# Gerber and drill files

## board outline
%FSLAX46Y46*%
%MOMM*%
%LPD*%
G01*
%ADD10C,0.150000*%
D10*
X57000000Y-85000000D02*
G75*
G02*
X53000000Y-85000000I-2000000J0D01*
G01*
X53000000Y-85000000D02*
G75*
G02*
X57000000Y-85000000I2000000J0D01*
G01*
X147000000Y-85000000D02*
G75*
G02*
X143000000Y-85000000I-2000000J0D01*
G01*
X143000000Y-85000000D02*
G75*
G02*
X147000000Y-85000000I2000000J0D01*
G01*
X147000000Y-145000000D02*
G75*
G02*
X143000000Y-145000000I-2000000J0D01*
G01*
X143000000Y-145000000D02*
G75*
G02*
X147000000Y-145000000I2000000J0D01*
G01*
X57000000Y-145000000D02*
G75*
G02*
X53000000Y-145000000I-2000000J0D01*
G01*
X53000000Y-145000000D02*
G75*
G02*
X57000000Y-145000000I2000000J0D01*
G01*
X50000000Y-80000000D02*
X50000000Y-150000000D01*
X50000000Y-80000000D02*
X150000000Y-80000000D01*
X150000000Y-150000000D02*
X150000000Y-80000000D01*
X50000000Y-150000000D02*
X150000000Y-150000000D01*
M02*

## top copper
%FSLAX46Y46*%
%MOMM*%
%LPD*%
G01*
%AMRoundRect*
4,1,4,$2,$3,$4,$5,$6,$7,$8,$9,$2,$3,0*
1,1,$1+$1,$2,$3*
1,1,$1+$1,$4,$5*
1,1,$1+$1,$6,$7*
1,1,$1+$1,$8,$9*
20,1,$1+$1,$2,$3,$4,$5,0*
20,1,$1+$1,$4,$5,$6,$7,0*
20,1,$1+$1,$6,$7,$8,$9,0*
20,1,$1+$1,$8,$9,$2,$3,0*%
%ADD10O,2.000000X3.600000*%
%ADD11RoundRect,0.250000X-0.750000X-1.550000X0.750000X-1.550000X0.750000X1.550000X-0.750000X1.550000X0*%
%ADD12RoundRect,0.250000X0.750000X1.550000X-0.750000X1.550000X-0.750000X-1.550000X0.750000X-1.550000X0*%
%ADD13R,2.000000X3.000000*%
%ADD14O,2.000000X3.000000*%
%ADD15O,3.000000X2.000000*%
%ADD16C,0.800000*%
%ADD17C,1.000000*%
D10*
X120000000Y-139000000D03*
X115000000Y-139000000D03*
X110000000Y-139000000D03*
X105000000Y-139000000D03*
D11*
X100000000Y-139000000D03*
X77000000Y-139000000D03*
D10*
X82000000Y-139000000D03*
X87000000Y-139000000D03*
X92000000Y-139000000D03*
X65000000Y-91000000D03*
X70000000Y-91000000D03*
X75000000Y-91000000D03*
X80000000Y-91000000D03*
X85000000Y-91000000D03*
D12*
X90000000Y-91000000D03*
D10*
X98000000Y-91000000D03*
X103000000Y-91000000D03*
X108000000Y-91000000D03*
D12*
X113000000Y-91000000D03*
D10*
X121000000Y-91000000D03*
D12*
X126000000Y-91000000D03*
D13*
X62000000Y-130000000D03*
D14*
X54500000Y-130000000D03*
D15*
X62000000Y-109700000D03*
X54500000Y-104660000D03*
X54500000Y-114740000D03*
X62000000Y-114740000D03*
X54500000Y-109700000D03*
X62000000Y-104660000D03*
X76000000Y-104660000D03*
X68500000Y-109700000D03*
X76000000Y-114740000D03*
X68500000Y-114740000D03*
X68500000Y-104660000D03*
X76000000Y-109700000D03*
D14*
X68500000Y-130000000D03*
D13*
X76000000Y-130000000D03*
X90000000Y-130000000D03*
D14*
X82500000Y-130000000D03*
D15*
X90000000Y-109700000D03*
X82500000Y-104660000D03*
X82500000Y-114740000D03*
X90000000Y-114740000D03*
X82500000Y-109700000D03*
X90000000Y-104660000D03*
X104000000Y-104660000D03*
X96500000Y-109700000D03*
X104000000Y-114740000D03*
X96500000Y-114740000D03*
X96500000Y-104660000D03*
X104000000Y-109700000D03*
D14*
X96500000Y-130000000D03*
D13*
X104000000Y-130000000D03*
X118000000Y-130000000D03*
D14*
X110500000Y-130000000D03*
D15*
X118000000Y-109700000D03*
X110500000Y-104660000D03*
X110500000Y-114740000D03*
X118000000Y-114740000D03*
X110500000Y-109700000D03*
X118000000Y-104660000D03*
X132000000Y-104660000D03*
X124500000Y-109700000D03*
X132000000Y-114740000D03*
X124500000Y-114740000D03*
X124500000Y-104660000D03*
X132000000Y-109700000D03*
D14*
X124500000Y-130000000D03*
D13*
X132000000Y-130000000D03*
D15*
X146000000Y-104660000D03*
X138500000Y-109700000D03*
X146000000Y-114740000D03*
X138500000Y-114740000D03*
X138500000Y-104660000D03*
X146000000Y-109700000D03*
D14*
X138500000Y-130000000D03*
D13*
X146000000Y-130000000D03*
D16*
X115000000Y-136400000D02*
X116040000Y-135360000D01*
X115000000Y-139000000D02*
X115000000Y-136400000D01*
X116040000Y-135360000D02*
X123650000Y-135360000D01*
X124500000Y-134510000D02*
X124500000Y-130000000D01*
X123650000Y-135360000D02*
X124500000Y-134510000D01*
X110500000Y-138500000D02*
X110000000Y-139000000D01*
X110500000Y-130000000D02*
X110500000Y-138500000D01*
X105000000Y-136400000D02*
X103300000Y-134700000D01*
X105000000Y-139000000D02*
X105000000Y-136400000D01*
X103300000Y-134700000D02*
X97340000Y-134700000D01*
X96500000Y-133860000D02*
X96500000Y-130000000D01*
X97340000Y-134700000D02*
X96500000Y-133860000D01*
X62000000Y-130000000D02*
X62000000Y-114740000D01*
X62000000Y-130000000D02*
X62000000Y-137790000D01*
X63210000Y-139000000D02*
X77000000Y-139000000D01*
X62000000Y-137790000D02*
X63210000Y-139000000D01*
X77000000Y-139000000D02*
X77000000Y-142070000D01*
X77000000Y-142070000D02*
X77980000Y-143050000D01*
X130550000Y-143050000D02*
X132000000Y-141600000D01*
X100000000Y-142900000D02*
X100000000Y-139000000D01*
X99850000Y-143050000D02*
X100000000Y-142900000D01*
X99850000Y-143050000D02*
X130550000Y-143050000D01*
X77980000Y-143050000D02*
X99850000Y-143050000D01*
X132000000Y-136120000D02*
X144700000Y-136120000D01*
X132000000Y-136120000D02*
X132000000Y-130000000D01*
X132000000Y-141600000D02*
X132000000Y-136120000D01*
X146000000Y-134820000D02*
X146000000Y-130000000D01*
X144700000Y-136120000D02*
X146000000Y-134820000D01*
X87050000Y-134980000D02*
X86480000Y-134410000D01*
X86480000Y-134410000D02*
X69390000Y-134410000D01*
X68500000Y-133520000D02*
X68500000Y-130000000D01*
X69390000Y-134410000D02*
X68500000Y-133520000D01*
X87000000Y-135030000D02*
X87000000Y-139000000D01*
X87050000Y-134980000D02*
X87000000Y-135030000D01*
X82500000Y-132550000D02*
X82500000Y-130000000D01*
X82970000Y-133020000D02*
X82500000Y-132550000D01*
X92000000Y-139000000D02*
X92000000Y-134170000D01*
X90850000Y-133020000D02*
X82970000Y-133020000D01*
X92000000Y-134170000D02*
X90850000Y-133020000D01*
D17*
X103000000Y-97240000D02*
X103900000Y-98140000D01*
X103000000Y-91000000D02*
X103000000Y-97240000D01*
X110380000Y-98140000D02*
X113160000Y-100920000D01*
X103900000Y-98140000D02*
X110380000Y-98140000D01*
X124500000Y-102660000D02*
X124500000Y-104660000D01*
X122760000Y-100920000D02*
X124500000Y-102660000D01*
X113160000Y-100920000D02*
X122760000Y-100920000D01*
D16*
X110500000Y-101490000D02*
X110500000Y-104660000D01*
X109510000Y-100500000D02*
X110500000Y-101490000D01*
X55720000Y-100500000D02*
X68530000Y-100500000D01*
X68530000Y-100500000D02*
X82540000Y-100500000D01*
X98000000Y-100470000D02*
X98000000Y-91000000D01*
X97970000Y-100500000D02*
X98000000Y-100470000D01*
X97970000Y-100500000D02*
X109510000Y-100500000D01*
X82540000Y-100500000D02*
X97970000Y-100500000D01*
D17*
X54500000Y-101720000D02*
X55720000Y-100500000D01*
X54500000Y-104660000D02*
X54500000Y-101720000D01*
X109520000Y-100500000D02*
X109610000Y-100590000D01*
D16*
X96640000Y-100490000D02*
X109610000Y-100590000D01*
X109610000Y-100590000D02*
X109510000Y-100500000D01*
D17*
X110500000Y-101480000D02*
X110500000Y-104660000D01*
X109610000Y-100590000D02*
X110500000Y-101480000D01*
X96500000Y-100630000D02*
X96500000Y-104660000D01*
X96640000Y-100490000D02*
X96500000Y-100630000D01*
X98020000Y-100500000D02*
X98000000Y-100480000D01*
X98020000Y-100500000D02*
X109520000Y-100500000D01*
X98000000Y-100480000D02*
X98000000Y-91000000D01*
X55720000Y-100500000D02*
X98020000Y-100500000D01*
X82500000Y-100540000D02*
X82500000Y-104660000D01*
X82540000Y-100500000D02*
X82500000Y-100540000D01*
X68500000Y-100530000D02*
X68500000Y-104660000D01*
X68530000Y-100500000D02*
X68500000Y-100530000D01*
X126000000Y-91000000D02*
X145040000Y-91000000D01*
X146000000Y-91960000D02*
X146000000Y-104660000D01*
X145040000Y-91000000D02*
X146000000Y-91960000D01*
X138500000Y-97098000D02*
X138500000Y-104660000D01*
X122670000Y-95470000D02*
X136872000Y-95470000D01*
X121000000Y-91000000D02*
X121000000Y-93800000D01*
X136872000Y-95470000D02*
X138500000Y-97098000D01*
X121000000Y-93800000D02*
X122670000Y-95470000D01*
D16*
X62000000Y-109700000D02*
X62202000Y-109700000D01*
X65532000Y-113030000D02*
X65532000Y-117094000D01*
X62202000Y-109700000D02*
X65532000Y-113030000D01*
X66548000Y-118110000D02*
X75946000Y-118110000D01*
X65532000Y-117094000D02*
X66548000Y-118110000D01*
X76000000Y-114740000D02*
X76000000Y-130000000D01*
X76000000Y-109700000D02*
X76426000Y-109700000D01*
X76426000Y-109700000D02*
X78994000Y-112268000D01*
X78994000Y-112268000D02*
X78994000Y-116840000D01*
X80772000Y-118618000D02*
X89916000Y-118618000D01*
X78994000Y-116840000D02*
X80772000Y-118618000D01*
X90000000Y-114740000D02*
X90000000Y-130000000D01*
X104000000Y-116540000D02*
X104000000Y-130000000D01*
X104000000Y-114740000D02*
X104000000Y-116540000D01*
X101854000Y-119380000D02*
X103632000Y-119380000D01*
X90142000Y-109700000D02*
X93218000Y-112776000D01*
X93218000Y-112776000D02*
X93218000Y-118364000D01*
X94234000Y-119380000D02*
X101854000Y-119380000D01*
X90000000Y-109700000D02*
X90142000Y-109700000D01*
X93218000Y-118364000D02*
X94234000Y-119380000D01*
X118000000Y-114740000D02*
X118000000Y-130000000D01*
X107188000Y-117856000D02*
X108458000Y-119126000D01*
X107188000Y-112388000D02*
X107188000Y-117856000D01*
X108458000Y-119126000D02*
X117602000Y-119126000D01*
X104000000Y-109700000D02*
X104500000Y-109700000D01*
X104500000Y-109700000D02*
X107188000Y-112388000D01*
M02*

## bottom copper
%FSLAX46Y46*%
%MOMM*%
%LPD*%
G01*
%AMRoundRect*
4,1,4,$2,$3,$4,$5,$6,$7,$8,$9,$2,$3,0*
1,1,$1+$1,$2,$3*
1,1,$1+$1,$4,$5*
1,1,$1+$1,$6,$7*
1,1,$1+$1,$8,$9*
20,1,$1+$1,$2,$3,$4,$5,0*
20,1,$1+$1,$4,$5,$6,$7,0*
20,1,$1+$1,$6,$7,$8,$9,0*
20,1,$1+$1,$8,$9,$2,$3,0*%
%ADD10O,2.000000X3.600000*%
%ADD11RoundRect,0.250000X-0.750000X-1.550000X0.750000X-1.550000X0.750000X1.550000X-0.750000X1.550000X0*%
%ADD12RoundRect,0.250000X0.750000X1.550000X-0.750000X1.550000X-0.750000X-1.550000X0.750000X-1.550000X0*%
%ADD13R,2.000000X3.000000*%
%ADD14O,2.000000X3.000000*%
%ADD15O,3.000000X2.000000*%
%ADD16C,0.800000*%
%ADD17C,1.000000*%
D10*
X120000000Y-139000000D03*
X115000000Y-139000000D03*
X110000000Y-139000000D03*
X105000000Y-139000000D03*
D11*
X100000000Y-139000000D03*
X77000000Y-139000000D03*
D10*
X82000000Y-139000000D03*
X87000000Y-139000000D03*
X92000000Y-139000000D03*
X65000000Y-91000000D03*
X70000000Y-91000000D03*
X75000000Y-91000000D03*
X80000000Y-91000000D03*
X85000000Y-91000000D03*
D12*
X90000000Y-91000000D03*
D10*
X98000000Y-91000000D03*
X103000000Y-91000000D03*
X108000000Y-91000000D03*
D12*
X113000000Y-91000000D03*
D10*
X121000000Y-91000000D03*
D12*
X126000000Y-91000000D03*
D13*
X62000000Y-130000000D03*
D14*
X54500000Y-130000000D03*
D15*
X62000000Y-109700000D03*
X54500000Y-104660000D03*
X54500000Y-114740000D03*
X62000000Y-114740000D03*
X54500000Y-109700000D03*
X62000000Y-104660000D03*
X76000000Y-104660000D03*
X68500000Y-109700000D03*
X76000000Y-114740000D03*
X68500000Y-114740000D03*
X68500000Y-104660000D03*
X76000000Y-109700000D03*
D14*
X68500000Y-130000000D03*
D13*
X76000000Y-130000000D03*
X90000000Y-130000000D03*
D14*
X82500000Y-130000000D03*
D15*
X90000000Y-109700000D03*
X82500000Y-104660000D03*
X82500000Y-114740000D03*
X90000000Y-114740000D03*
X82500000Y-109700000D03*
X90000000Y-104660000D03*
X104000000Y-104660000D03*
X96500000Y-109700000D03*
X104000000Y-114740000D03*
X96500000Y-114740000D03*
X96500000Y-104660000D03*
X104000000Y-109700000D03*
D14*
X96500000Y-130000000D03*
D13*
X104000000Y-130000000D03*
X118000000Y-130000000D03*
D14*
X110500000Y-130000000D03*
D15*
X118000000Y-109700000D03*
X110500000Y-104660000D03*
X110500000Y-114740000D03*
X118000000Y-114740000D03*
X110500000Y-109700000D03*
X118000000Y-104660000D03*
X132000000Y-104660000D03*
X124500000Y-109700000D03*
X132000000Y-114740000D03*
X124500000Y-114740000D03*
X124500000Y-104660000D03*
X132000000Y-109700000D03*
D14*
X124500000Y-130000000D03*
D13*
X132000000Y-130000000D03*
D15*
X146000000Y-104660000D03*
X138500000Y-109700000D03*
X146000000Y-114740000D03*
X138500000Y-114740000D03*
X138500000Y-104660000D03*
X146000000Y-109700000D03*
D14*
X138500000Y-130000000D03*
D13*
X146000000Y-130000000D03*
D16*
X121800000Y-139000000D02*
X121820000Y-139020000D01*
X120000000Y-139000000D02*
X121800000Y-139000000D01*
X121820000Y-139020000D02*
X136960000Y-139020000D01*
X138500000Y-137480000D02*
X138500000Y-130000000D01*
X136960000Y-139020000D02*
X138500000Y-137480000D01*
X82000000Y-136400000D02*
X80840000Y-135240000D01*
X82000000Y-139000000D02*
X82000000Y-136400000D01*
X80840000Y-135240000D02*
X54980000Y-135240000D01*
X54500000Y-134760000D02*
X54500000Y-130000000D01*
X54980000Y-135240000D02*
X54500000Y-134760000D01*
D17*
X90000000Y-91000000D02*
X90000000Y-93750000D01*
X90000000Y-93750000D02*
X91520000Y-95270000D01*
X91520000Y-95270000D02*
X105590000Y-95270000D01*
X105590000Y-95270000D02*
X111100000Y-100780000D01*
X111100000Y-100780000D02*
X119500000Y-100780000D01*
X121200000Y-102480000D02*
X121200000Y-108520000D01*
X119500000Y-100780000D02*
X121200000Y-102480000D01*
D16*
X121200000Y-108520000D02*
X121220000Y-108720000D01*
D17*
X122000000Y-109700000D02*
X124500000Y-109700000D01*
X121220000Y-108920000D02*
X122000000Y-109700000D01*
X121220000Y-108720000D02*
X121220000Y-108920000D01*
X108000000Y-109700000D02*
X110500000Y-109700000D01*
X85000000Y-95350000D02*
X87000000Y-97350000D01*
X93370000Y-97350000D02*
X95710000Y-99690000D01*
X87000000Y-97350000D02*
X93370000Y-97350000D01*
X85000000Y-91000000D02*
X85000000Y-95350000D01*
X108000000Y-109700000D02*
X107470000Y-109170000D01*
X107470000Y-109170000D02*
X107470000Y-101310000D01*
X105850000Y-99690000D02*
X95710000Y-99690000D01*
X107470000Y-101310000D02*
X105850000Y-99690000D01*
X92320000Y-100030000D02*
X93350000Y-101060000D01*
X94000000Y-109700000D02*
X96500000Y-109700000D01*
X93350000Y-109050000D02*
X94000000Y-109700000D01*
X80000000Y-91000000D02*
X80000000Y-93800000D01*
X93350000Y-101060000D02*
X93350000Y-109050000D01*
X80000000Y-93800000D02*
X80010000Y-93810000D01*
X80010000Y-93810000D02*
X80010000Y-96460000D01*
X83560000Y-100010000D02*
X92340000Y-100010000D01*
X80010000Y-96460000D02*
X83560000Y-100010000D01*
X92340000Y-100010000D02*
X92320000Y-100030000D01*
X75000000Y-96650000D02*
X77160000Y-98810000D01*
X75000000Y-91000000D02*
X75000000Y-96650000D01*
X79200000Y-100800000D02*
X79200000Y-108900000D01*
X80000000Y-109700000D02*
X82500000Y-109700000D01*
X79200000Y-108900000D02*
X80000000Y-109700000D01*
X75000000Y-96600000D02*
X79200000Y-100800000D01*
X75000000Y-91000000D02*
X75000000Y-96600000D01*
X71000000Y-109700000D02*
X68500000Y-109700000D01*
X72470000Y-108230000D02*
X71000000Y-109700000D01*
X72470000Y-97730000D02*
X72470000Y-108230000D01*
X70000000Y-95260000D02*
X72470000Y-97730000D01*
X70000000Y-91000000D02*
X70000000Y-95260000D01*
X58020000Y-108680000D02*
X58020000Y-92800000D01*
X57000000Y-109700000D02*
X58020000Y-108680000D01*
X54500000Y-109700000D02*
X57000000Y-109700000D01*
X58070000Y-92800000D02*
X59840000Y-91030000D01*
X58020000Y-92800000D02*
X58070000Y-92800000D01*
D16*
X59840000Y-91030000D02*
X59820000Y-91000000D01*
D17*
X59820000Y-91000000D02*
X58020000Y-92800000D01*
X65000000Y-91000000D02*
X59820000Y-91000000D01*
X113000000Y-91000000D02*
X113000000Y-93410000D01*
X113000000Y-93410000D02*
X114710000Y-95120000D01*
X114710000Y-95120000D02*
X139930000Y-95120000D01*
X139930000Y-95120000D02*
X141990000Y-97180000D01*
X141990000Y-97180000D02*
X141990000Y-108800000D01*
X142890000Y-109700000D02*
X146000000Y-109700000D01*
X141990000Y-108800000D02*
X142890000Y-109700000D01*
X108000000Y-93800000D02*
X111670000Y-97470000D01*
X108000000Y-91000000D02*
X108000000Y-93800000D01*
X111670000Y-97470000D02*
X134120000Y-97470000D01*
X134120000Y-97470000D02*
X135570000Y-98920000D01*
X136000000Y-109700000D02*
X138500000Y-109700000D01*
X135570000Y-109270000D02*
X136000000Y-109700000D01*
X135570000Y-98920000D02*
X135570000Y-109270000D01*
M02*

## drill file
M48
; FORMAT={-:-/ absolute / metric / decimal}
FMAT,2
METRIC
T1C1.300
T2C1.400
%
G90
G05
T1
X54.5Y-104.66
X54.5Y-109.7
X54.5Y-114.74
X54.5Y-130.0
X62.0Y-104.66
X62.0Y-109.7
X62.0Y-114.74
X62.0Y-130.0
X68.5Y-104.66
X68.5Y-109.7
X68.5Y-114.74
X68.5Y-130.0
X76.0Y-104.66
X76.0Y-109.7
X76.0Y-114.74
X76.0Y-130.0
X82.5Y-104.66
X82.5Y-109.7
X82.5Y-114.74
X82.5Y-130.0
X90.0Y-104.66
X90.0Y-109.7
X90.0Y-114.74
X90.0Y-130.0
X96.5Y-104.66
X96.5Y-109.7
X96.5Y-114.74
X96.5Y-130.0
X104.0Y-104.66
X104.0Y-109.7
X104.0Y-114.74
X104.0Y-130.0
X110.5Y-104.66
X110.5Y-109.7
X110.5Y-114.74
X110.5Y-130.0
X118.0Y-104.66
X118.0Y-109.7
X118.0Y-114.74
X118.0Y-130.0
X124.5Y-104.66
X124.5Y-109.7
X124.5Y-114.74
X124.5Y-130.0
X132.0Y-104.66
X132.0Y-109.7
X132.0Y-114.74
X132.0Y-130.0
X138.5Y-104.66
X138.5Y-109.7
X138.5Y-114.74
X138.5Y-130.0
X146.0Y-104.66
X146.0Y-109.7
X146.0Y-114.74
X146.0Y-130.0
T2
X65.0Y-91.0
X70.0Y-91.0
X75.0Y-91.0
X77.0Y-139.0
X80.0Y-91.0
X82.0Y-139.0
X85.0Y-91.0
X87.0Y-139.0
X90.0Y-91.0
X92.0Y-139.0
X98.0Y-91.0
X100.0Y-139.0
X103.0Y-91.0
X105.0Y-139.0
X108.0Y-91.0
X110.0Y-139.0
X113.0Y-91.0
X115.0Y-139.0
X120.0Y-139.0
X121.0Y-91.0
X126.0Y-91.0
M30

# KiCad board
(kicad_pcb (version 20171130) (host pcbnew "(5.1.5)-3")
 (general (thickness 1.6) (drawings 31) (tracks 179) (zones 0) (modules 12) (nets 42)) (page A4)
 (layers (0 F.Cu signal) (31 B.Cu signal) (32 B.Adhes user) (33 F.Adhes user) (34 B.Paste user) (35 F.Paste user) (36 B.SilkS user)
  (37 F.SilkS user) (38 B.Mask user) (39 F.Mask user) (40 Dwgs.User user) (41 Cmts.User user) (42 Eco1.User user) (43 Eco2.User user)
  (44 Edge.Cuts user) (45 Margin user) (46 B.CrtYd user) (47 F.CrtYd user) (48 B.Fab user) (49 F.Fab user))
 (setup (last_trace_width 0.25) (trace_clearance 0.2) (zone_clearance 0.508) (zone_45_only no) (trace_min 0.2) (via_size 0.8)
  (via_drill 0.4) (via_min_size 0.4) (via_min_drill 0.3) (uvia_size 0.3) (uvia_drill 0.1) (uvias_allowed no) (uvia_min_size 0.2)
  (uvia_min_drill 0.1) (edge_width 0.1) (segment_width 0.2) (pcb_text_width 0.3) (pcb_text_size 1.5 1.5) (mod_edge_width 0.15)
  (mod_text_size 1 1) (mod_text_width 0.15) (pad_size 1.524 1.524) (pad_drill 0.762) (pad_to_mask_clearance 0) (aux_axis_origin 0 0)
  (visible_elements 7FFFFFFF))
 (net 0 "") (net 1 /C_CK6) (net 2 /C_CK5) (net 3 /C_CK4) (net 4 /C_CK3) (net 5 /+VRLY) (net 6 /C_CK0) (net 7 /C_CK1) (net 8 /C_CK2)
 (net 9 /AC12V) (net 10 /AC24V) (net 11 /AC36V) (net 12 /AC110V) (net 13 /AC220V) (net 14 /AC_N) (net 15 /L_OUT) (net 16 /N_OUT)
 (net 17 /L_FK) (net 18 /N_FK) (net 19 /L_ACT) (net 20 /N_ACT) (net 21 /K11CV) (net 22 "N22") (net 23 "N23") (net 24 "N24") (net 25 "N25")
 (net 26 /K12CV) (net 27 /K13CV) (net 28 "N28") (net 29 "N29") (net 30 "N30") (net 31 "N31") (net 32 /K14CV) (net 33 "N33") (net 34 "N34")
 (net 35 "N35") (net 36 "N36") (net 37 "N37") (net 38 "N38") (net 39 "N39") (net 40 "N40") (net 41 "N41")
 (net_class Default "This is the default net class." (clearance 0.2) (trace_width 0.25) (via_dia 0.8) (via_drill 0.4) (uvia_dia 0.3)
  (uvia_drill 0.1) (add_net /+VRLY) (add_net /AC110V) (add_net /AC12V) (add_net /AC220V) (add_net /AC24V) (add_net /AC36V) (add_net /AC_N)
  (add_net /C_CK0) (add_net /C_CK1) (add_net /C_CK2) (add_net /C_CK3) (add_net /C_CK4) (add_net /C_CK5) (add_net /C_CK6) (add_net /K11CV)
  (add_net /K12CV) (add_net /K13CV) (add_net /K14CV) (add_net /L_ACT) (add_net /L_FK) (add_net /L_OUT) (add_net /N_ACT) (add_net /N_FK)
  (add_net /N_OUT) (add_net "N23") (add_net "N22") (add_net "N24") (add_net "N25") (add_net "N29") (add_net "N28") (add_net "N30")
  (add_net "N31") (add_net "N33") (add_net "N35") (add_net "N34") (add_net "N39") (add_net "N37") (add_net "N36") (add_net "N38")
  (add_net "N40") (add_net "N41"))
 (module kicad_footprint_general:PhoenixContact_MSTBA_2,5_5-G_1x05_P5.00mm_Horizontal (layer F.Cu) (at 100 139)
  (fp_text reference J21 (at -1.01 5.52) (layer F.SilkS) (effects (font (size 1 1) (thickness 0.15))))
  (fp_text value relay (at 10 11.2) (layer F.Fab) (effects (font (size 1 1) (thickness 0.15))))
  (pad 5 thru_hole oval (at 20 0) (size 2 3.6) (drill 1.4) (layers *.Cu *.Mask) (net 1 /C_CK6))
  (pad 4 thru_hole oval (at 15 0) (size 2 3.6) (drill 1.4) (layers *.Cu *.Mask) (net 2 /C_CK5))
  (pad 3 thru_hole oval (at 10 0) (size 2 3.6) (drill 1.4) (layers *.Cu *.Mask) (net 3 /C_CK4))
  (pad 2 thru_hole oval (at 5 0) (size 2 3.6) (drill 1.4) (layers *.Cu *.Mask) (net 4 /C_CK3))
  (pad 1 thru_hole roundrect (at 0 0) (size 2 3.6) (drill 1.4) (layers *.Cu *.Mask) (roundrect_rratio 0.125) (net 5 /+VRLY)))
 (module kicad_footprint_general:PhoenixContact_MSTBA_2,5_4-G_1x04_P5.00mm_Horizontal (layer F.Cu) (at 77 139)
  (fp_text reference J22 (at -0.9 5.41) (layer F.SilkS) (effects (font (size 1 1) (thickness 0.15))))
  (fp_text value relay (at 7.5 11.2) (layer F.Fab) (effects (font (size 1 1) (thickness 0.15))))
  (pad 1 thru_hole roundrect (at 0 0) (size 2 3.6) (drill 1.4) (layers *.Cu *.Mask) (roundrect_rratio 0.125) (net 5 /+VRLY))
  (pad 2 thru_hole oval (at 5 0) (size 2 3.6) (drill 1.4) (layers *.Cu *.Mask) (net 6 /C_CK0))
  (pad 3 thru_hole oval (at 10 0) (size 2 3.6) (drill 1.4) (layers *.Cu *.Mask) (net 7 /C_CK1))
  (pad 4 thru_hole oval (at 15 0) (size 2 3.6) (drill 1.4) (layers *.Cu *.Mask) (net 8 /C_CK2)))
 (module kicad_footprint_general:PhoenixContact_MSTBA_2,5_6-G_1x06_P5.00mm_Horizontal (layer F.Cu) (at 90 91 180)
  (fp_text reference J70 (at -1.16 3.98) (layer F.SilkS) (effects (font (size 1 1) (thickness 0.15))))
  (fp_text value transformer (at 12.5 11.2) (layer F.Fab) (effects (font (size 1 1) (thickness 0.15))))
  (pad 6 thru_hole oval (at 25 0 180) (size 2 3.6) (drill 1.4) (layers *.Cu *.Mask) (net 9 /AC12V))
  (pad 5 thru_hole oval (at 20 0 180) (size 2 3.6) (drill 1.4) (layers *.Cu *.Mask) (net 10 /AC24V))
  (pad 4 thru_hole oval (at 15 0 180) (size 2 3.6) (drill 1.4) (layers *.Cu *.Mask) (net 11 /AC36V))
  (pad 3 thru_hole oval (at 10 0 180) (size 2 3.6) (drill 1.4) (layers *.Cu *.Mask) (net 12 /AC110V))
  (pad 2 thru_hole oval (at 5 0 180) (size 2 3.6) (drill 1.4) (layers *.Cu *.Mask) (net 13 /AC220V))
  (pad 1 thru_hole roundrect (at 0 0 180) (size 2 3.6) (drill 1.4) (layers *.Cu *.Mask) (roundrect_rratio 0.125) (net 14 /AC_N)))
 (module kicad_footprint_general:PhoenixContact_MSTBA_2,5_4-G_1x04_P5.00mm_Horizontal (layer F.Cu) (at 113 91 180)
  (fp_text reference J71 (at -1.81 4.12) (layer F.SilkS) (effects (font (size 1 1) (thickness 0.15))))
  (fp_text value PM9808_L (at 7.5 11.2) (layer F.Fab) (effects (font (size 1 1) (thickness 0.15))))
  (pad 4 thru_hole oval (at 15 0 180) (size 2 3.6) (drill 1.4) (layers *.Cu *.Mask) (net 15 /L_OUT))
  (pad 3 thru_hole oval (at 10 0 180) (size 2 3.6) (drill 1.4) (layers *.Cu *.Mask) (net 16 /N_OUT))
  (pad 2 thru_hole oval (at 5 0 180) (size 2 3.6) (drill 1.4) (layers *.Cu *.Mask) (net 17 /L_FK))
  (pad 1 thru_hole roundrect (at 0 0 180) (size 2 3.6) (drill 1.4) (layers *.Cu *.Mask) (roundrect_rratio 0.125) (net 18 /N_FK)))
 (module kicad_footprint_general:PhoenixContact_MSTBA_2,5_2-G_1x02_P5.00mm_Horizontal (layer F.Cu) (at 126 91 180)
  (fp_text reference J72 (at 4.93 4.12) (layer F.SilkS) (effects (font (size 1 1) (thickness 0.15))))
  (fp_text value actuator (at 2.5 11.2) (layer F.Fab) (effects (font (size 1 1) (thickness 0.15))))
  (pad 2 thru_hole oval (at 5 0 180) (size 2 3.6) (drill 1.4) (layers *.Cu *.Mask) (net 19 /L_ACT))
  (pad 1 thru_hole roundrect (at 0 0 180) (size 2 3.6) (drill 1.4) (layers *.Cu *.Mask) (roundrect_rratio 0.125) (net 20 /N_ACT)))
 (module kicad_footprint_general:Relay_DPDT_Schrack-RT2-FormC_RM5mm (layer F.Cu) (at 62 130 90)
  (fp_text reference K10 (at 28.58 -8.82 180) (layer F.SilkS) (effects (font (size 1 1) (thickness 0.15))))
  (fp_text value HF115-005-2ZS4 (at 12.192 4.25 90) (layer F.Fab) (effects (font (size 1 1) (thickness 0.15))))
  (pad A1 thru_hole rect (at 0 0 270) (size 3 2) (drill 1.3) (layers *.Cu *.Mask) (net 5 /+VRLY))
  (pad A2 thru_hole oval (at 0 -7.5 270) (size 3 2) (drill 1.3) (layers *.Cu *.Mask) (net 6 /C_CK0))
  (pad 11 thru_hole oval (at 20.3 0 270) (size 2 3) (drill 1.3) (layers *.Cu *.Mask) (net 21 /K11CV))
  (pad 24 thru_hole oval (at 25.34 -7.5 270) (size 2 3) (drill 1.3) (layers *.Cu *.Mask) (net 15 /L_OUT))
  (pad 22 thru_hole oval (at 15.26 -7.5 270) (size 2 3) (drill 1.3) (layers *.Cu *.Mask) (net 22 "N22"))
  (pad 12 thru_hole oval (at 15.26 0 270) (size 2 3) (drill 1.3) (layers *.Cu *.Mask) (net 5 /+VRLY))
  (pad 21 thru_hole oval (at 20.3 -7.5 270) (size 2 3) (drill 1.3) (layers *.Cu *.Mask) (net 9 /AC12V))
  (pad 14 thru_hole oval (at 25.34 0 270) (size 2 3) (drill 1.3) (layers *.Cu *.Mask) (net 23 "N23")))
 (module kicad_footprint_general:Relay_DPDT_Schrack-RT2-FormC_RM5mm (layer F.Cu) (at 76 130 90)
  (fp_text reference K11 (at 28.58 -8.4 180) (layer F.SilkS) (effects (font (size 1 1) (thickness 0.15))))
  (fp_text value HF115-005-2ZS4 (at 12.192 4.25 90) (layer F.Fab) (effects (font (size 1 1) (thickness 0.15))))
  (pad 14 thru_hole oval (at 25.34 0 270) (size 2 3) (drill 1.3) (layers *.Cu *.Mask) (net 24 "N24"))
  (pad 21 thru_hole oval (at 20.3 -7.5 270) (size 2 3) (drill 1.3) (layers *.Cu *.Mask) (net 10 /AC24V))
  (pad 12 thru_hole oval (at 15.26 0 270) (size 2 3) (drill 1.3) (layers *.Cu *.Mask) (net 21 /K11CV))
  (pad 22 thru_hole oval (at 15.26 -7.5 270) (size 2 3) (drill 1.3) (layers *.Cu *.Mask) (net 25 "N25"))
  (pad 24 thru_hole oval (at 25.34 -7.5 270) (size 2 3) (drill 1.3) (layers *.Cu *.Mask) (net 15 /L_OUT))
  (pad 11 thru_hole oval (at 20.3 0 270) (size 2 3) (drill 1.3) (layers *.Cu *.Mask) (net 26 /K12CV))
  (pad A2 thru_hole oval (at 0 -7.5 270) (size 3 2) (drill 1.3) (layers *.Cu *.Mask) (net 7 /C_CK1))
  (pad A1 thru_hole rect (at 0 0 270) (size 3 2) (drill 1.3) (layers *.Cu *.Mask) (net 21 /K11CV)))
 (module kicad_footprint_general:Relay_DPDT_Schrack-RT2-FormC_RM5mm (layer F.Cu) (at 90 130 90)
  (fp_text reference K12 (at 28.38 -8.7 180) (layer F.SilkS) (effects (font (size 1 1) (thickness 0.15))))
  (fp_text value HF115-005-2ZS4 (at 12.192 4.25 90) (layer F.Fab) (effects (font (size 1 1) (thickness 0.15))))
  (pad A1 thru_hole rect (at 0 0 270) (size 3 2) (drill 1.3) (layers *.Cu *.Mask) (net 26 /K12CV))
  (pad A2 thru_hole oval (at 0 -7.5 270) (size 3 2) (drill 1.3) (layers *.Cu *.Mask) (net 8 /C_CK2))
  (pad 11 thru_hole oval (at 20.3 0 270) (size 2 3) (drill 1.3) (layers *.Cu *.Mask) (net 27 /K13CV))
  (pad 24 thru_hole oval (at 25.34 -7.5 270) (size 2 3) (drill 1.3) (layers *.Cu *.Mask) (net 15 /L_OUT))
  (pad 22 thru_hole oval (at 15.26 -7.5 270) (size 2 3) (drill 1.3) (layers *.Cu *.Mask) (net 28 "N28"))
  (pad 12 thru_hole oval (at 15.26 0 270) (size 2 3) (drill 1.3) (layers *.Cu *.Mask) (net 26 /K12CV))
  (pad 21 thru_hole oval (at 20.3 -7.5 270) (size 2 3) (drill 1.3) (layers *.Cu *.Mask) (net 11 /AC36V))
  (pad 14 thru_hole oval (at 25.34 0 270) (size 2 3) (drill 1.3) (layers *.Cu *.Mask) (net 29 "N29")))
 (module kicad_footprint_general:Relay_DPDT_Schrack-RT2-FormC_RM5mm (layer F.Cu) (at 104 130 90)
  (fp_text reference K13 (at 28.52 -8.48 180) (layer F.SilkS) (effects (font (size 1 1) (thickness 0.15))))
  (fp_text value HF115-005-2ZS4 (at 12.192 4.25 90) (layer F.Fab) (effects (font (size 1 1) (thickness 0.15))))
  (pad 14 thru_hole oval (at 25.34 0 270) (size 2 3) (drill 1.3) (layers *.Cu *.Mask) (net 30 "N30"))
  (pad 21 thru_hole oval (at 20.3 -7.5 270) (size 2 3) (drill 1.3) (layers *.Cu *.Mask) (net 12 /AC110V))
  (pad 12 thru_hole oval (at 15.26 0 270) (size 2 3) (drill 1.3) (layers *.Cu *.Mask) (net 27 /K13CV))
  (pad 22 thru_hole oval (at 15.26 -7.5 270) (size 2 3) (drill 1.3) (layers *.Cu *.Mask) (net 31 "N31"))
  (pad 24 thru_hole oval (at 25.34 -7.5 270) (size 2 3) (drill 1.3) (layers *.Cu *.Mask) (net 15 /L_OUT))
  (pad 11 thru_hole oval (at 20.3 0 270) (size 2 3) (drill 1.3) (layers *.Cu *.Mask) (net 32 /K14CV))
  (pad A2 thru_hole oval (at 0 -7.5 270) (size 3 2) (drill 1.3) (layers *.Cu *.Mask) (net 4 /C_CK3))
  (pad A1 thru_hole rect (at 0 0 270) (size 3 2) (drill 1.3) (layers *.Cu *.Mask) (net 27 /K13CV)))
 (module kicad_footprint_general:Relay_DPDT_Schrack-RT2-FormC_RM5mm (layer F.Cu) (at 118 130 90)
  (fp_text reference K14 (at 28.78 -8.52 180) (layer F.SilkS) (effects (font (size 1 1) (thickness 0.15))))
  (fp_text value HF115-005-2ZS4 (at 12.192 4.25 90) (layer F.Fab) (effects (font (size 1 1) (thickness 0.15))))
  (pad A1 thru_hole rect (at 0 0 270) (size 3 2) (drill 1.3) (layers *.Cu *.Mask) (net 32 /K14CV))
  (pad A2 thru_hole oval (at 0 -7.5 270) (size 3 2) (drill 1.3) (layers *.Cu *.Mask) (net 3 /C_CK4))
  (pad 11 thru_hole oval (at 20.3 0 270) (size 2 3) (drill 1.3) (layers *.Cu *.Mask) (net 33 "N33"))
  (pad 24 thru_hole oval (at 25.34 -7.5 270) (size 2 3) (drill 1.3) (layers *.Cu *.Mask) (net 15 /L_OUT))
  (pad 22 thru_hole oval (at 15.26 -7.5 270) (size 2 3) (drill 1.3) (layers *.Cu *.Mask) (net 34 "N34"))
  (pad 12 thru_hole oval (at 15.26 0 270) (size 2 3) (drill 1.3) (layers *.Cu *.Mask) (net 32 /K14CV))
  (pad 21 thru_hole oval (at 20.3 -7.5 270) (size 2 3) (drill 1.3) (layers *.Cu *.Mask) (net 13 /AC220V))
  (pad 14 thru_hole oval (at 25.34 0 270) (size 2 3) (drill 1.3) (layers *.Cu *.Mask) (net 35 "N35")))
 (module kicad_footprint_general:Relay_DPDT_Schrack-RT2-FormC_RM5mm (layer F.Cu) (at 132 130 90)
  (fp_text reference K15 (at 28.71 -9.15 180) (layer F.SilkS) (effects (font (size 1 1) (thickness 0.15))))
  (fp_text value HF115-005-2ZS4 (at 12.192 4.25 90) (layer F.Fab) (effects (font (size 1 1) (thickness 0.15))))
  (pad 14 thru_hole oval (at 25.34 0 270) (size 2 3) (drill 1.3) (layers *.Cu *.Mask) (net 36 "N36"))
  (pad 21 thru_hole oval (at 20.3 -7.5 270) (size 2 3) (drill 1.3) (layers *.Cu *.Mask) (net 14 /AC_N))
  (pad 12 thru_hole oval (at 15.26 0 270) (size 2 3) (drill 1.3) (layers *.Cu *.Mask) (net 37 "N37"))
  (pad 22 thru_hole oval (at 15.26 -7.5 270) (size 2 3) (drill 1.3) (layers *.Cu *.Mask) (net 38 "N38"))
  (pad 24 thru_hole oval (at 25.34 -7.5 270) (size 2 3) (drill 1.3) (layers *.Cu *.Mask) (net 16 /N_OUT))
  (pad 11 thru_hole oval (at 20.3 0 270) (size 2 3) (drill 1.3) (layers *.Cu *.Mask) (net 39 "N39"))
  (pad A2 thru_hole oval (at 0 -7.5 270) (size 3 2) (drill 1.3) (layers *.Cu *.Mask) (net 2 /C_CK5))
  (pad A1 thru_hole rect (at 0 0 270) (size 3 2) (drill 1.3) (layers *.Cu *.Mask) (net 5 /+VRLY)))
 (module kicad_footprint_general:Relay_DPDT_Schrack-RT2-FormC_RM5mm (layer F.Cu) (at 146 130 90)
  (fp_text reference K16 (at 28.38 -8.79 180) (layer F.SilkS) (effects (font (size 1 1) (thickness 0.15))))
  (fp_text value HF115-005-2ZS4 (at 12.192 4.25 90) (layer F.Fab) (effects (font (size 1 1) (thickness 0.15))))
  (pad 14 thru_hole oval (at 25.34 0 270) (size 2 3) (drill 1.3) (layers *.Cu *.Mask) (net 20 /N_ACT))
  (pad 21 thru_hole oval (at 20.3 -7.5 270) (size 2 3) (drill 1.3) (layers *.Cu *.Mask) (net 17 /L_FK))
  (pad 12 thru_hole oval (at 15.26 0 270) (size 2 3) (drill 1.3) (layers *.Cu *.Mask) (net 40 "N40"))
  (pad 22 thru_hole oval (at 15.26 -7.5 270) (size 2 3) (drill 1.3) (layers *.Cu *.Mask) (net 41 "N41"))
  (pad 24 thru_hole oval (at 25.34 -7.5 270) (size 2 3) (drill 1.3) (layers *.Cu *.Mask) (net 19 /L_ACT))
  (pad 11 thru_hole oval (at 20.3 0 270) (size 2 3) (drill 1.3) (layers *.Cu *.Mask) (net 18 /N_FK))
  (pad A2 thru_hole oval (at 0 -7.5 270) (size 3 2) (drill 1.3) (layers *.Cu *.Mask) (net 1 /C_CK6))
  (pad A1 thru_hole rect (at 0 0 270) (size 3 2) (drill 1.3) (layers *.Cu *.Mask) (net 5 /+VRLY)))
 (gr_circle (center 55 85) (end 57 85) (layer Edge.Cuts) (width 0.15))
 (gr_circle (center 145 85) (end 147 85) (layer Edge.Cuts) (width 0.15))
 (gr_circle (center 145 145) (end 147 145) (layer Edge.Cuts) (width 0.15))
 (gr_circle (center 55 145) (end 57 145) (layer Edge.Cuts) (width 0.15))
 (gr_line (start 50 80) (end 50 150) (layer Edge.Cuts) (width 0.15))
 (gr_line (start 50 80) (end 150 80) (layer Edge.Cuts) (width 0.15))
 (gr_line (start 150 150) (end 150 80) (layer Edge.Cuts) (width 0.15))
 (gr_line (start 50 150) (end 150 150) (layer Edge.Cuts) (width 0.15))
 (segment (start 121.8 139) (end 121.82 139.02) (width 0.8) (layer B.Cu) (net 1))
 (segment (start 120 139) (end 121.8 139) (width 0.8) (layer B.Cu) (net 1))
 (segment (start 121.82 139.02) (end 136.96 139.02) (width 0.8) (layer B.Cu) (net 1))
 (segment (start 138.5 137.48) (end 138.5 130) (width 0.8) (layer B.Cu) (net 1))
 (segment (start 136.96 139.02) (end 138.5 137.48) (width 0.8) (layer B.Cu) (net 1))
 (segment (start 115 136.4) (end 116.04 135.36) (width 0.8) (layer F.Cu) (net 2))
 (segment (start 115 139) (end 115 136.4) (width 0.8) (layer F.Cu) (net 2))
 (segment (start 116.04 135.36) (end 123.65 135.36) (width 0.8) (layer F.Cu) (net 2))
 (segment (start 124.5 134.51) (end 124.5 130) (width 0.8) (layer F.Cu) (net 2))
 (segment (start 123.65 135.36) (end 124.5 134.51) (width 0.8) (layer F.Cu) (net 2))
 (segment (start 110.5 138.5) (end 110 139) (width 0.8) (layer F.Cu) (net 3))
 (segment (start 110.5 130) (end 110.5 138.5) (width 0.8) (layer F.Cu) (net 3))
 (segment (start 105 136.4) (end 103.3 134.7) (width 0.8) (layer F.Cu) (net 4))
 (segment (start 105 139) (end 105 136.4) (width 0.8) (layer F.Cu) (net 4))
 (segment (start 103.3 134.7) (end 97.34 134.7) (width 0.8) (layer F.Cu) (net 4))
 (segment (start 96.5 133.86) (end 96.5 130) (width 0.8) (layer F.Cu) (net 4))
 (segment (start 97.34 134.7) (end 96.5 133.86) (width 0.8) (layer F.Cu) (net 4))
 (segment (start 62 130) (end 62 114.74) (width 0.8) (layer F.Cu) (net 5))
 (segment (start 62 130) (end 62 137.79) (width 0.8) (layer F.Cu) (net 5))
 (segment (start 63.21 139) (end 77 139) (width 0.8) (layer F.Cu) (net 5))
 (segment (start 62 137.79) (end 63.21 139) (width 0.8) (layer F.Cu) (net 5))
 (segment (start 77 139) (end 77 142.07) (width 0.8) (layer F.Cu) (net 5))
 (segment (start 77 142.07) (end 77.98 143.05) (width 0.8) (layer F.Cu) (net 5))
 (segment (start 130.55 143.05) (end 132 141.6) (width 0.8) (layer F.Cu) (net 5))
 (segment (start 100 142.9) (end 100 139) (width 0.8) (layer F.Cu) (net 5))
 (segment (start 99.85 143.05) (end 100 142.9) (width 0.8) (layer F.Cu) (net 5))
 (segment (start 99.85 143.05) (end 130.55 143.05) (width 0.8) (layer F.Cu) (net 5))
 (segment (start 77.98 143.05) (end 99.85 143.05) (width 0.8) (layer F.Cu) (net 5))
 (segment (start 132 136.12) (end 144.7 136.12) (width 0.8) (layer F.Cu) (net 5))
 (segment (start 132 136.12) (end 132 130) (width 0.8) (layer F.Cu) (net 5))
 (segment (start 132 141.6) (end 132 136.12) (width 0.8) (layer F.Cu) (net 5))
 (segment (start 146 134.82) (end 146 130) (width 0.8) (layer F.Cu) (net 5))
 (segment (start 144.7 136.12) (end 146 134.82) (width 0.8) (layer F.Cu) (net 5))
 (segment (start 82 136.4) (end 80.84 135.24) (width 0.8) (layer B.Cu) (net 6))
 (segment (start 82 139) (end 82 136.4) (width 0.8) (layer B.Cu) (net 6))
 (segment (start 80.84 135.24) (end 54.98 135.24) (width 0.8) (layer B.Cu) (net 6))
 (segment (start 54.5 134.76) (end 54.5 130) (width 0.8) (layer B.Cu) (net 6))
 (segment (start 54.98 135.24) (end 54.5 134.76) (width 0.8) (layer B.Cu) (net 6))
 (segment (start 87.05 134.98) (end 86.48 134.41) (width 0.8) (layer F.Cu) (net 7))
 (segment (start 86.48 134.41) (end 69.39 134.41) (width 0.8) (layer F.Cu) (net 7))
 (segment (start 68.5 133.52) (end 68.5 130) (width 0.8) (layer F.Cu) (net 7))
 (segment (start 69.39 134.41) (end 68.5 133.52) (width 0.8) (layer F.Cu) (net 7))
 (segment (start 87 135.03) (end 87 139) (width 0.8) (layer F.Cu) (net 7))
 (segment (start 87.05 134.98) (end 87 135.03) (width 0.8) (layer F.Cu) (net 7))
 (segment (start 82.5 132.55) (end 82.5 130) (width 0.8) (layer F.Cu) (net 8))
 (segment (start 82.97 133.02) (end 82.5 132.55) (width 0.8) (layer F.Cu) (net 8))
 (segment (start 92 139) (end 92 134.17) (width 0.8) (layer F.Cu) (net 8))
 (segment (start 90.85 133.02) (end 82.97 133.02) (width 0.8) (layer F.Cu) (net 8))
 (segment (start 92 134.17) (end 90.85 133.02) (width 0.8) (layer F.Cu) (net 8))
 (segment (start 90 91) (end 90 93.75) (width 1) (layer B.Cu) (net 14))
 (segment (start 90 93.75) (end 91.52 95.27) (width 1) (layer B.Cu) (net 14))
 (segment (start 91.52 95.27) (end 105.59 95.27) (width 1) (layer B.Cu) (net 14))
 (segment (start 105.59 95.27) (end 111.1 100.78) (width 1) (layer B.Cu) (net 14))
 (segment (start 111.1 100.78) (end 119.5 100.78) (width 1) (layer B.Cu) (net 14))
 (segment (start 121.2 102.48) (end 121.2 108.52) (width 1) (layer B.Cu) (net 14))
 (segment (start 119.5 100.78) (end 121.2 102.48) (width 1) (layer B.Cu) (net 14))
 (segment (start 121.2 108.52) (end 121.22 108.72) (width 0.8) (layer B.Cu) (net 14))
 (segment (start 122 109.7) (end 124.5 109.7) (width 1) (layer B.Cu) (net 14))
 (segment (start 121.22 108.92) (end 122 109.7) (width 1) (layer B.Cu) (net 14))
 (segment (start 121.22 108.72) (end 121.22 108.92) (width 1) (layer B.Cu) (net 14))
 (segment (start 108 109.7) (end 110.5 109.7) (width 1) (layer B.Cu) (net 13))
 (segment (start 85 95.35) (end 87 97.35) (width 1) (layer B.Cu) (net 13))
 (segment (start 93.37 97.35) (end 95.71 99.69) (width 1) (layer B.Cu) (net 13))
 (segment (start 87 97.35) (end 93.37 97.35) (width 1) (layer B.Cu) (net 13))
 (segment (start 85 91) (end 85 95.35) (width 1) (layer B.Cu) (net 13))
 (segment (start 108 109.7) (end 107.47 109.17) (width 1) (layer B.Cu) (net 13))
 (segment (start 107.47 109.17) (end 107.47 101.31) (width 1) (layer B.Cu) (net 13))
 (segment (start 105.85 99.69) (end 95.71 99.69) (width 1) (layer B.Cu) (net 13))
 (segment (start 107.47 101.31) (end 105.85 99.69) (width 1) (layer B.Cu) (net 13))
 (segment (start 92.32 100.03) (end 93.35 101.06) (width 1) (layer B.Cu) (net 12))
 (segment (start 94 109.7) (end 96.5 109.7) (width 1) (layer B.Cu) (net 12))
 (segment (start 93.35 109.05) (end 94 109.7) (width 1) (layer B.Cu) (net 12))
 (segment (start 80 91) (end 80 93.8) (width 1) (layer B.Cu) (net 12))
 (segment (start 93.35 101.06) (end 93.35 109.05) (width 1) (layer B.Cu) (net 12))
 (segment (start 80 93.8) (end 80.01 93.81) (width 1) (layer B.Cu) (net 12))
 (segment (start 80.01 93.81) (end 80.01 96.46) (width 1) (layer B.Cu) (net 12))
 (segment (start 83.56 100.01) (end 92.34 100.01) (width 1) (layer B.Cu) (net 12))
 (segment (start 80.01 96.46) (end 83.56 100.01) (width 1) (layer B.Cu) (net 12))
 (segment (start 92.34 100.01) (end 92.32 100.03) (width 1) (layer B.Cu) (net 12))
 (segment (start 75 96.65) (end 77.16 98.81) (width 1) (layer B.Cu) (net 11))
 (segment (start 75 91) (end 75 96.65) (width 1) (layer B.Cu) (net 11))
 (segment (start 79.2 100.8) (end 79.2 108.9) (width 1) (layer B.Cu) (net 11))
 (segment (start 80 109.7) (end 82.5 109.7) (width 1) (layer B.Cu) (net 11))
 (segment (start 79.2 108.9) (end 80 109.7) (width 1) (layer B.Cu) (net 11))
 (segment (start 75 96.6) (end 79.2 100.8) (width 1) (layer B.Cu) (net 11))
 (segment (start 75 91) (end 75 96.6) (width 1) (layer B.Cu) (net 11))
 (segment (start 71 109.7) (end 68.5 109.7) (width 1) (layer B.Cu) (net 10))
 (segment (start 72.47 108.23) (end 71 109.7) (width 1) (layer B.Cu) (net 10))
 (segment (start 72.47 97.73) (end 72.47 108.23) (width 1) (layer B.Cu) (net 10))
 (segment (start 70 95.26) (end 72.47 97.73) (width 1) (layer B.Cu) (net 10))
 (segment (start 70 91) (end 70 95.26) (width 1) (layer B.Cu) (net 10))
 (segment (start 58.02 108.68) (end 58.02 92.8) (width 1) (layer B.Cu) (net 9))
 (segment (start 57 109.7) (end 58.02 108.68) (width 1) (layer B.Cu) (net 9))
 (segment (start 54.5 109.7) (end 57 109.7) (width 1) (layer B.Cu) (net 9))
 (segment (start 58.07 92.8) (end 59.84 91.03) (width 1) (layer B.Cu) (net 9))
 (segment (start 58.02 92.8) (end 58.07 92.8) (width 1) (layer B.Cu) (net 9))
 (segment (start 59.84 91.03) (end 59.82 91) (width 0.8) (layer B.Cu) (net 9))
 (segment (start 59.82 91) (end 58.02 92.8) (width 1) (layer B.Cu) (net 9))
 (segment (start 65 91) (end 59.82 91) (width 1) (layer B.Cu) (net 9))
 (segment (start 113 91) (end 113 93.41) (width 1) (layer B.Cu) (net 18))
 (segment (start 113 93.41) (end 114.71 95.12) (width 1) (layer B.Cu) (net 18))
 (segment (start 114.71 95.12) (end 139.93 95.12) (width 1) (layer B.Cu) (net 18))
 (segment (start 139.93 95.12) (end 141.99 97.18) (width 1) (layer B.Cu) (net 18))
 (segment (start 141.99 97.18) (end 141.99 108.8) (width 1) (layer B.Cu) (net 18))
 (segment (start 142.89 109.7) (end 146 109.7) (width 1) (layer B.Cu) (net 18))
 (segment (start 141.99 108.8) (end 142.89 109.7) (width 1) (layer B.Cu) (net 18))
 (segment (start 108 93.8) (end 111.67 97.47) (width 1) (layer B.Cu) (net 17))
 (segment (start 108 91) (end 108 93.8) (width 1) (layer B.Cu) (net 17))
 (segment (start 111.67 97.47) (end 134.12 97.47) (width 1) (layer B.Cu) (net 17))
 (segment (start 134.12 97.47) (end 135.57 98.92) (width 1) (layer B.Cu) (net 17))
 (segment (start 136 109.7) (end 138.5 109.7) (width 1) (layer B.Cu) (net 17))
 (segment (start 135.57 109.27) (end 136 109.7) (width 1) (layer B.Cu) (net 17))
 (segment (start 135.57 98.92) (end 135.57 109.27) (width 1) (layer B.Cu) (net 17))
 (segment (start 103 97.24) (end 103.9 98.14) (width 1) (layer F.Cu) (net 16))
 (segment (start 103 91) (end 103 97.24) (width 1) (layer F.Cu) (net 16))
 (segment (start 110.38 98.14) (end 113.16 100.92) (width 1) (layer F.Cu) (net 16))
 (segment (start 103.9 98.14) (end 110.38 98.14) (width 1) (layer F.Cu) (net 16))
 (segment (start 124.5 102.66) (end 124.5 104.66) (width 1) (layer F.Cu) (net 16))
 (segment (start 122.76 100.92) (end 124.5 102.66) (width 1) (layer F.Cu) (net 16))
 (segment (start 113.16 100.92) (end 122.76 100.92) (width 1) (layer F.Cu) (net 16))
 (segment (start 110.5 101.49) (end 110.5 104.66) (width 0.8) (layer F.Cu) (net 15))
 (segment (start 109.51 100.5) (end 110.5 101.49) (width 0.8) (layer F.Cu) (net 15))
 (segment (start 55.72 100.5) (end 68.53 100.5) (width 0.8) (layer F.Cu) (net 15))
 (segment (start 68.53 100.5) (end 82.54 100.5) (width 0.8) (layer F.Cu) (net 15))
 (segment (start 98 100.47) (end 98 91) (width 0.8) (layer F.Cu) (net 15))
 (segment (start 97.97 100.5) (end 98 100.47) (width 0.8) (layer F.Cu) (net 15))
 (segment (start 97.97 100.5) (end 109.51 100.5) (width 0.8) (layer F.Cu) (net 15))
 (segment (start 82.54 100.5) (end 97.97 100.5) (width 0.8) (layer F.Cu) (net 15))
 (segment (start 54.5 101.72) (end 55.72 100.5) (width 1) (layer F.Cu) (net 15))
 (segment (start 54.5 104.66) (end 54.5 101.72) (width 1) (layer F.Cu) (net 15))
 (segment (start 109.52 100.5) (end 109.61 100.59) (width 1) (layer F.Cu) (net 15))
 (segment (start 96.64 100.49) (end 109.61 100.59) (width 0.8) (layer F.Cu) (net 15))
 (segment (start 109.61 100.59) (end 109.51 100.5) (width 0.8) (layer F.Cu) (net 15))
 (segment (start 110.5 101.48) (end 110.5 104.66) (width 1) (layer F.Cu) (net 15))
 (segment (start 109.61 100.59) (end 110.5 101.48) (width 1) (layer F.Cu) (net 15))
 (segment (start 96.5 100.63) (end 96.5 104.66) (width 1) (layer F.Cu) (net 15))
 (segment (start 96.64 100.49) (end 96.5 100.63) (width 1) (layer F.Cu) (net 15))
 (segment (start 98.02 100.5) (end 98 100.48) (width 1) (layer F.Cu) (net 15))
 (segment (start 98.02 100.5) (end 109.52 100.5) (width 1) (layer F.Cu) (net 15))
 (segment (start 98 100.48) (end 98 91) (width 1) (layer F.Cu) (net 15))
 (segment (start 55.72 100.5) (end 98.02 100.5) (width 1) (layer F.Cu) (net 15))
 (segment (start 82.5 100.54) (end 82.5 104.66) (width 1) (layer F.Cu) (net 15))
 (segment (start 82.54 100.5) (end 82.5 100.54) (width 1) (layer F.Cu) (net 15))
 (segment (start 68.5 100.53) (end 68.5 104.66) (width 1) (layer F.Cu) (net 15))
 (segment (start 68.53 100.5) (end 68.5 100.53) (width 1) (layer F.Cu) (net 15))
 (segment (start 126 91) (end 145.04 91) (width 1) (layer F.Cu) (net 20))
 (segment (start 146 91.96) (end 146 104.66) (width 1) (layer F.Cu) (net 20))
 (segment (start 145.04 91) (end 146 91.96) (width 1) (layer F.Cu) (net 20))
 (segment (start 138.5 97.098) (end 138.5 104.66) (width 1) (layer F.Cu) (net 19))
 (segment (start 122.67 95.47) (end 136.872 95.47) (width 1) (layer F.Cu) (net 19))
 (segment (start 121 91) (end 121 93.8) (width 1) (layer F.Cu) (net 19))
 (segment (start 136.872 95.47) (end 138.5 97.098) (width 1) (layer F.Cu) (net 19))
 (segment (start 121 93.8) (end 122.67 95.47) (width 1) (layer F.Cu) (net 19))
 (segment (start 62 109.7) (end 62.202 109.7) (width 0.8) (layer F.Cu) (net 21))
 (segment (start 65.532 113.03) (end 65.532 117.094) (width 0.8) (layer F.Cu) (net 21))
 (segment (start 62.202 109.7) (end 65.532 113.03) (width 0.8) (layer F.Cu) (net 21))
 (segment (start 66.548 118.11) (end 75.946 118.11) (width 0.8) (layer F.Cu) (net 21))
 (segment (start 65.532 117.094) (end 66.548 118.11) (width 0.8) (layer F.Cu) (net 21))
 (segment (start 76 114.74) (end 76 130) (width 0.8) (layer F.Cu) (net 21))
 (segment (start 76 109.7) (end 76.426 109.7) (width 0.8) (layer F.Cu) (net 26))
 (segment (start 76.426 109.7) (end 78.994 112.268) (width 0.8) (layer F.Cu) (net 26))
 (segment (start 78.994 112.268) (end 78.994 116.84) (width 0.8) (layer F.Cu) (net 26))
 (segment (start 80.772 118.618) (end 89.916 118.618) (width 0.8) (layer F.Cu) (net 26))
 (segment (start 78.994 116.84) (end 80.772 118.618) (width 0.8) (layer F.Cu) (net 26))
 (segment (start 90 114.74) (end 90 130) (width 0.8) (layer F.Cu) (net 26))
 (segment (start 104 116.54) (end 104 130) (width 0.8) (layer F.Cu) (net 27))
 (segment (start 104 114.74) (end 104 116.54) (width 0.8) (layer F.Cu) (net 27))
 (segment (start 101.854 119.38) (end 103.632 119.38) (width 0.8) (layer F.Cu) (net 27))
 (segment (start 90.142 109.7) (end 93.218 112.776) (width 0.8) (layer F.Cu) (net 27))
 (segment (start 93.218 112.776) (end 93.218 118.364) (width 0.8) (layer F.Cu) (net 27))
 (segment (start 94.234 119.38) (end 101.854 119.38) (width 0.8) (layer F.Cu) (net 27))
 (segment (start 90 109.7) (end 90.142 109.7) (width 0.8) (layer F.Cu) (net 27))
 (segment (start 93.218 118.364) (end 94.234 119.38) (width 0.8) (layer F.Cu) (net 27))
 (segment (start 118 114.74) (end 118 130) (width 0.8) (layer F.Cu) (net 32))
 (segment (start 107.188 117.856) (end 108.458 119.126) (width 0.8) (layer F.Cu) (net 32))
 (segment (start 107.188 112.388) (end 107.188 117.856) (width 0.8) (layer F.Cu) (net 32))
 (segment (start 108.458 119.126) (end 117.602 119.126) (width 0.8) (layer F.Cu) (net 32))
 (segment (start 104 109.7) (end 104.5 109.7) (width 0.8) (layer F.Cu) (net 32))
 (segment (start 104.5 109.7) (end 107.188 112.388) (width 0.8) (layer F.Cu) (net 32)))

